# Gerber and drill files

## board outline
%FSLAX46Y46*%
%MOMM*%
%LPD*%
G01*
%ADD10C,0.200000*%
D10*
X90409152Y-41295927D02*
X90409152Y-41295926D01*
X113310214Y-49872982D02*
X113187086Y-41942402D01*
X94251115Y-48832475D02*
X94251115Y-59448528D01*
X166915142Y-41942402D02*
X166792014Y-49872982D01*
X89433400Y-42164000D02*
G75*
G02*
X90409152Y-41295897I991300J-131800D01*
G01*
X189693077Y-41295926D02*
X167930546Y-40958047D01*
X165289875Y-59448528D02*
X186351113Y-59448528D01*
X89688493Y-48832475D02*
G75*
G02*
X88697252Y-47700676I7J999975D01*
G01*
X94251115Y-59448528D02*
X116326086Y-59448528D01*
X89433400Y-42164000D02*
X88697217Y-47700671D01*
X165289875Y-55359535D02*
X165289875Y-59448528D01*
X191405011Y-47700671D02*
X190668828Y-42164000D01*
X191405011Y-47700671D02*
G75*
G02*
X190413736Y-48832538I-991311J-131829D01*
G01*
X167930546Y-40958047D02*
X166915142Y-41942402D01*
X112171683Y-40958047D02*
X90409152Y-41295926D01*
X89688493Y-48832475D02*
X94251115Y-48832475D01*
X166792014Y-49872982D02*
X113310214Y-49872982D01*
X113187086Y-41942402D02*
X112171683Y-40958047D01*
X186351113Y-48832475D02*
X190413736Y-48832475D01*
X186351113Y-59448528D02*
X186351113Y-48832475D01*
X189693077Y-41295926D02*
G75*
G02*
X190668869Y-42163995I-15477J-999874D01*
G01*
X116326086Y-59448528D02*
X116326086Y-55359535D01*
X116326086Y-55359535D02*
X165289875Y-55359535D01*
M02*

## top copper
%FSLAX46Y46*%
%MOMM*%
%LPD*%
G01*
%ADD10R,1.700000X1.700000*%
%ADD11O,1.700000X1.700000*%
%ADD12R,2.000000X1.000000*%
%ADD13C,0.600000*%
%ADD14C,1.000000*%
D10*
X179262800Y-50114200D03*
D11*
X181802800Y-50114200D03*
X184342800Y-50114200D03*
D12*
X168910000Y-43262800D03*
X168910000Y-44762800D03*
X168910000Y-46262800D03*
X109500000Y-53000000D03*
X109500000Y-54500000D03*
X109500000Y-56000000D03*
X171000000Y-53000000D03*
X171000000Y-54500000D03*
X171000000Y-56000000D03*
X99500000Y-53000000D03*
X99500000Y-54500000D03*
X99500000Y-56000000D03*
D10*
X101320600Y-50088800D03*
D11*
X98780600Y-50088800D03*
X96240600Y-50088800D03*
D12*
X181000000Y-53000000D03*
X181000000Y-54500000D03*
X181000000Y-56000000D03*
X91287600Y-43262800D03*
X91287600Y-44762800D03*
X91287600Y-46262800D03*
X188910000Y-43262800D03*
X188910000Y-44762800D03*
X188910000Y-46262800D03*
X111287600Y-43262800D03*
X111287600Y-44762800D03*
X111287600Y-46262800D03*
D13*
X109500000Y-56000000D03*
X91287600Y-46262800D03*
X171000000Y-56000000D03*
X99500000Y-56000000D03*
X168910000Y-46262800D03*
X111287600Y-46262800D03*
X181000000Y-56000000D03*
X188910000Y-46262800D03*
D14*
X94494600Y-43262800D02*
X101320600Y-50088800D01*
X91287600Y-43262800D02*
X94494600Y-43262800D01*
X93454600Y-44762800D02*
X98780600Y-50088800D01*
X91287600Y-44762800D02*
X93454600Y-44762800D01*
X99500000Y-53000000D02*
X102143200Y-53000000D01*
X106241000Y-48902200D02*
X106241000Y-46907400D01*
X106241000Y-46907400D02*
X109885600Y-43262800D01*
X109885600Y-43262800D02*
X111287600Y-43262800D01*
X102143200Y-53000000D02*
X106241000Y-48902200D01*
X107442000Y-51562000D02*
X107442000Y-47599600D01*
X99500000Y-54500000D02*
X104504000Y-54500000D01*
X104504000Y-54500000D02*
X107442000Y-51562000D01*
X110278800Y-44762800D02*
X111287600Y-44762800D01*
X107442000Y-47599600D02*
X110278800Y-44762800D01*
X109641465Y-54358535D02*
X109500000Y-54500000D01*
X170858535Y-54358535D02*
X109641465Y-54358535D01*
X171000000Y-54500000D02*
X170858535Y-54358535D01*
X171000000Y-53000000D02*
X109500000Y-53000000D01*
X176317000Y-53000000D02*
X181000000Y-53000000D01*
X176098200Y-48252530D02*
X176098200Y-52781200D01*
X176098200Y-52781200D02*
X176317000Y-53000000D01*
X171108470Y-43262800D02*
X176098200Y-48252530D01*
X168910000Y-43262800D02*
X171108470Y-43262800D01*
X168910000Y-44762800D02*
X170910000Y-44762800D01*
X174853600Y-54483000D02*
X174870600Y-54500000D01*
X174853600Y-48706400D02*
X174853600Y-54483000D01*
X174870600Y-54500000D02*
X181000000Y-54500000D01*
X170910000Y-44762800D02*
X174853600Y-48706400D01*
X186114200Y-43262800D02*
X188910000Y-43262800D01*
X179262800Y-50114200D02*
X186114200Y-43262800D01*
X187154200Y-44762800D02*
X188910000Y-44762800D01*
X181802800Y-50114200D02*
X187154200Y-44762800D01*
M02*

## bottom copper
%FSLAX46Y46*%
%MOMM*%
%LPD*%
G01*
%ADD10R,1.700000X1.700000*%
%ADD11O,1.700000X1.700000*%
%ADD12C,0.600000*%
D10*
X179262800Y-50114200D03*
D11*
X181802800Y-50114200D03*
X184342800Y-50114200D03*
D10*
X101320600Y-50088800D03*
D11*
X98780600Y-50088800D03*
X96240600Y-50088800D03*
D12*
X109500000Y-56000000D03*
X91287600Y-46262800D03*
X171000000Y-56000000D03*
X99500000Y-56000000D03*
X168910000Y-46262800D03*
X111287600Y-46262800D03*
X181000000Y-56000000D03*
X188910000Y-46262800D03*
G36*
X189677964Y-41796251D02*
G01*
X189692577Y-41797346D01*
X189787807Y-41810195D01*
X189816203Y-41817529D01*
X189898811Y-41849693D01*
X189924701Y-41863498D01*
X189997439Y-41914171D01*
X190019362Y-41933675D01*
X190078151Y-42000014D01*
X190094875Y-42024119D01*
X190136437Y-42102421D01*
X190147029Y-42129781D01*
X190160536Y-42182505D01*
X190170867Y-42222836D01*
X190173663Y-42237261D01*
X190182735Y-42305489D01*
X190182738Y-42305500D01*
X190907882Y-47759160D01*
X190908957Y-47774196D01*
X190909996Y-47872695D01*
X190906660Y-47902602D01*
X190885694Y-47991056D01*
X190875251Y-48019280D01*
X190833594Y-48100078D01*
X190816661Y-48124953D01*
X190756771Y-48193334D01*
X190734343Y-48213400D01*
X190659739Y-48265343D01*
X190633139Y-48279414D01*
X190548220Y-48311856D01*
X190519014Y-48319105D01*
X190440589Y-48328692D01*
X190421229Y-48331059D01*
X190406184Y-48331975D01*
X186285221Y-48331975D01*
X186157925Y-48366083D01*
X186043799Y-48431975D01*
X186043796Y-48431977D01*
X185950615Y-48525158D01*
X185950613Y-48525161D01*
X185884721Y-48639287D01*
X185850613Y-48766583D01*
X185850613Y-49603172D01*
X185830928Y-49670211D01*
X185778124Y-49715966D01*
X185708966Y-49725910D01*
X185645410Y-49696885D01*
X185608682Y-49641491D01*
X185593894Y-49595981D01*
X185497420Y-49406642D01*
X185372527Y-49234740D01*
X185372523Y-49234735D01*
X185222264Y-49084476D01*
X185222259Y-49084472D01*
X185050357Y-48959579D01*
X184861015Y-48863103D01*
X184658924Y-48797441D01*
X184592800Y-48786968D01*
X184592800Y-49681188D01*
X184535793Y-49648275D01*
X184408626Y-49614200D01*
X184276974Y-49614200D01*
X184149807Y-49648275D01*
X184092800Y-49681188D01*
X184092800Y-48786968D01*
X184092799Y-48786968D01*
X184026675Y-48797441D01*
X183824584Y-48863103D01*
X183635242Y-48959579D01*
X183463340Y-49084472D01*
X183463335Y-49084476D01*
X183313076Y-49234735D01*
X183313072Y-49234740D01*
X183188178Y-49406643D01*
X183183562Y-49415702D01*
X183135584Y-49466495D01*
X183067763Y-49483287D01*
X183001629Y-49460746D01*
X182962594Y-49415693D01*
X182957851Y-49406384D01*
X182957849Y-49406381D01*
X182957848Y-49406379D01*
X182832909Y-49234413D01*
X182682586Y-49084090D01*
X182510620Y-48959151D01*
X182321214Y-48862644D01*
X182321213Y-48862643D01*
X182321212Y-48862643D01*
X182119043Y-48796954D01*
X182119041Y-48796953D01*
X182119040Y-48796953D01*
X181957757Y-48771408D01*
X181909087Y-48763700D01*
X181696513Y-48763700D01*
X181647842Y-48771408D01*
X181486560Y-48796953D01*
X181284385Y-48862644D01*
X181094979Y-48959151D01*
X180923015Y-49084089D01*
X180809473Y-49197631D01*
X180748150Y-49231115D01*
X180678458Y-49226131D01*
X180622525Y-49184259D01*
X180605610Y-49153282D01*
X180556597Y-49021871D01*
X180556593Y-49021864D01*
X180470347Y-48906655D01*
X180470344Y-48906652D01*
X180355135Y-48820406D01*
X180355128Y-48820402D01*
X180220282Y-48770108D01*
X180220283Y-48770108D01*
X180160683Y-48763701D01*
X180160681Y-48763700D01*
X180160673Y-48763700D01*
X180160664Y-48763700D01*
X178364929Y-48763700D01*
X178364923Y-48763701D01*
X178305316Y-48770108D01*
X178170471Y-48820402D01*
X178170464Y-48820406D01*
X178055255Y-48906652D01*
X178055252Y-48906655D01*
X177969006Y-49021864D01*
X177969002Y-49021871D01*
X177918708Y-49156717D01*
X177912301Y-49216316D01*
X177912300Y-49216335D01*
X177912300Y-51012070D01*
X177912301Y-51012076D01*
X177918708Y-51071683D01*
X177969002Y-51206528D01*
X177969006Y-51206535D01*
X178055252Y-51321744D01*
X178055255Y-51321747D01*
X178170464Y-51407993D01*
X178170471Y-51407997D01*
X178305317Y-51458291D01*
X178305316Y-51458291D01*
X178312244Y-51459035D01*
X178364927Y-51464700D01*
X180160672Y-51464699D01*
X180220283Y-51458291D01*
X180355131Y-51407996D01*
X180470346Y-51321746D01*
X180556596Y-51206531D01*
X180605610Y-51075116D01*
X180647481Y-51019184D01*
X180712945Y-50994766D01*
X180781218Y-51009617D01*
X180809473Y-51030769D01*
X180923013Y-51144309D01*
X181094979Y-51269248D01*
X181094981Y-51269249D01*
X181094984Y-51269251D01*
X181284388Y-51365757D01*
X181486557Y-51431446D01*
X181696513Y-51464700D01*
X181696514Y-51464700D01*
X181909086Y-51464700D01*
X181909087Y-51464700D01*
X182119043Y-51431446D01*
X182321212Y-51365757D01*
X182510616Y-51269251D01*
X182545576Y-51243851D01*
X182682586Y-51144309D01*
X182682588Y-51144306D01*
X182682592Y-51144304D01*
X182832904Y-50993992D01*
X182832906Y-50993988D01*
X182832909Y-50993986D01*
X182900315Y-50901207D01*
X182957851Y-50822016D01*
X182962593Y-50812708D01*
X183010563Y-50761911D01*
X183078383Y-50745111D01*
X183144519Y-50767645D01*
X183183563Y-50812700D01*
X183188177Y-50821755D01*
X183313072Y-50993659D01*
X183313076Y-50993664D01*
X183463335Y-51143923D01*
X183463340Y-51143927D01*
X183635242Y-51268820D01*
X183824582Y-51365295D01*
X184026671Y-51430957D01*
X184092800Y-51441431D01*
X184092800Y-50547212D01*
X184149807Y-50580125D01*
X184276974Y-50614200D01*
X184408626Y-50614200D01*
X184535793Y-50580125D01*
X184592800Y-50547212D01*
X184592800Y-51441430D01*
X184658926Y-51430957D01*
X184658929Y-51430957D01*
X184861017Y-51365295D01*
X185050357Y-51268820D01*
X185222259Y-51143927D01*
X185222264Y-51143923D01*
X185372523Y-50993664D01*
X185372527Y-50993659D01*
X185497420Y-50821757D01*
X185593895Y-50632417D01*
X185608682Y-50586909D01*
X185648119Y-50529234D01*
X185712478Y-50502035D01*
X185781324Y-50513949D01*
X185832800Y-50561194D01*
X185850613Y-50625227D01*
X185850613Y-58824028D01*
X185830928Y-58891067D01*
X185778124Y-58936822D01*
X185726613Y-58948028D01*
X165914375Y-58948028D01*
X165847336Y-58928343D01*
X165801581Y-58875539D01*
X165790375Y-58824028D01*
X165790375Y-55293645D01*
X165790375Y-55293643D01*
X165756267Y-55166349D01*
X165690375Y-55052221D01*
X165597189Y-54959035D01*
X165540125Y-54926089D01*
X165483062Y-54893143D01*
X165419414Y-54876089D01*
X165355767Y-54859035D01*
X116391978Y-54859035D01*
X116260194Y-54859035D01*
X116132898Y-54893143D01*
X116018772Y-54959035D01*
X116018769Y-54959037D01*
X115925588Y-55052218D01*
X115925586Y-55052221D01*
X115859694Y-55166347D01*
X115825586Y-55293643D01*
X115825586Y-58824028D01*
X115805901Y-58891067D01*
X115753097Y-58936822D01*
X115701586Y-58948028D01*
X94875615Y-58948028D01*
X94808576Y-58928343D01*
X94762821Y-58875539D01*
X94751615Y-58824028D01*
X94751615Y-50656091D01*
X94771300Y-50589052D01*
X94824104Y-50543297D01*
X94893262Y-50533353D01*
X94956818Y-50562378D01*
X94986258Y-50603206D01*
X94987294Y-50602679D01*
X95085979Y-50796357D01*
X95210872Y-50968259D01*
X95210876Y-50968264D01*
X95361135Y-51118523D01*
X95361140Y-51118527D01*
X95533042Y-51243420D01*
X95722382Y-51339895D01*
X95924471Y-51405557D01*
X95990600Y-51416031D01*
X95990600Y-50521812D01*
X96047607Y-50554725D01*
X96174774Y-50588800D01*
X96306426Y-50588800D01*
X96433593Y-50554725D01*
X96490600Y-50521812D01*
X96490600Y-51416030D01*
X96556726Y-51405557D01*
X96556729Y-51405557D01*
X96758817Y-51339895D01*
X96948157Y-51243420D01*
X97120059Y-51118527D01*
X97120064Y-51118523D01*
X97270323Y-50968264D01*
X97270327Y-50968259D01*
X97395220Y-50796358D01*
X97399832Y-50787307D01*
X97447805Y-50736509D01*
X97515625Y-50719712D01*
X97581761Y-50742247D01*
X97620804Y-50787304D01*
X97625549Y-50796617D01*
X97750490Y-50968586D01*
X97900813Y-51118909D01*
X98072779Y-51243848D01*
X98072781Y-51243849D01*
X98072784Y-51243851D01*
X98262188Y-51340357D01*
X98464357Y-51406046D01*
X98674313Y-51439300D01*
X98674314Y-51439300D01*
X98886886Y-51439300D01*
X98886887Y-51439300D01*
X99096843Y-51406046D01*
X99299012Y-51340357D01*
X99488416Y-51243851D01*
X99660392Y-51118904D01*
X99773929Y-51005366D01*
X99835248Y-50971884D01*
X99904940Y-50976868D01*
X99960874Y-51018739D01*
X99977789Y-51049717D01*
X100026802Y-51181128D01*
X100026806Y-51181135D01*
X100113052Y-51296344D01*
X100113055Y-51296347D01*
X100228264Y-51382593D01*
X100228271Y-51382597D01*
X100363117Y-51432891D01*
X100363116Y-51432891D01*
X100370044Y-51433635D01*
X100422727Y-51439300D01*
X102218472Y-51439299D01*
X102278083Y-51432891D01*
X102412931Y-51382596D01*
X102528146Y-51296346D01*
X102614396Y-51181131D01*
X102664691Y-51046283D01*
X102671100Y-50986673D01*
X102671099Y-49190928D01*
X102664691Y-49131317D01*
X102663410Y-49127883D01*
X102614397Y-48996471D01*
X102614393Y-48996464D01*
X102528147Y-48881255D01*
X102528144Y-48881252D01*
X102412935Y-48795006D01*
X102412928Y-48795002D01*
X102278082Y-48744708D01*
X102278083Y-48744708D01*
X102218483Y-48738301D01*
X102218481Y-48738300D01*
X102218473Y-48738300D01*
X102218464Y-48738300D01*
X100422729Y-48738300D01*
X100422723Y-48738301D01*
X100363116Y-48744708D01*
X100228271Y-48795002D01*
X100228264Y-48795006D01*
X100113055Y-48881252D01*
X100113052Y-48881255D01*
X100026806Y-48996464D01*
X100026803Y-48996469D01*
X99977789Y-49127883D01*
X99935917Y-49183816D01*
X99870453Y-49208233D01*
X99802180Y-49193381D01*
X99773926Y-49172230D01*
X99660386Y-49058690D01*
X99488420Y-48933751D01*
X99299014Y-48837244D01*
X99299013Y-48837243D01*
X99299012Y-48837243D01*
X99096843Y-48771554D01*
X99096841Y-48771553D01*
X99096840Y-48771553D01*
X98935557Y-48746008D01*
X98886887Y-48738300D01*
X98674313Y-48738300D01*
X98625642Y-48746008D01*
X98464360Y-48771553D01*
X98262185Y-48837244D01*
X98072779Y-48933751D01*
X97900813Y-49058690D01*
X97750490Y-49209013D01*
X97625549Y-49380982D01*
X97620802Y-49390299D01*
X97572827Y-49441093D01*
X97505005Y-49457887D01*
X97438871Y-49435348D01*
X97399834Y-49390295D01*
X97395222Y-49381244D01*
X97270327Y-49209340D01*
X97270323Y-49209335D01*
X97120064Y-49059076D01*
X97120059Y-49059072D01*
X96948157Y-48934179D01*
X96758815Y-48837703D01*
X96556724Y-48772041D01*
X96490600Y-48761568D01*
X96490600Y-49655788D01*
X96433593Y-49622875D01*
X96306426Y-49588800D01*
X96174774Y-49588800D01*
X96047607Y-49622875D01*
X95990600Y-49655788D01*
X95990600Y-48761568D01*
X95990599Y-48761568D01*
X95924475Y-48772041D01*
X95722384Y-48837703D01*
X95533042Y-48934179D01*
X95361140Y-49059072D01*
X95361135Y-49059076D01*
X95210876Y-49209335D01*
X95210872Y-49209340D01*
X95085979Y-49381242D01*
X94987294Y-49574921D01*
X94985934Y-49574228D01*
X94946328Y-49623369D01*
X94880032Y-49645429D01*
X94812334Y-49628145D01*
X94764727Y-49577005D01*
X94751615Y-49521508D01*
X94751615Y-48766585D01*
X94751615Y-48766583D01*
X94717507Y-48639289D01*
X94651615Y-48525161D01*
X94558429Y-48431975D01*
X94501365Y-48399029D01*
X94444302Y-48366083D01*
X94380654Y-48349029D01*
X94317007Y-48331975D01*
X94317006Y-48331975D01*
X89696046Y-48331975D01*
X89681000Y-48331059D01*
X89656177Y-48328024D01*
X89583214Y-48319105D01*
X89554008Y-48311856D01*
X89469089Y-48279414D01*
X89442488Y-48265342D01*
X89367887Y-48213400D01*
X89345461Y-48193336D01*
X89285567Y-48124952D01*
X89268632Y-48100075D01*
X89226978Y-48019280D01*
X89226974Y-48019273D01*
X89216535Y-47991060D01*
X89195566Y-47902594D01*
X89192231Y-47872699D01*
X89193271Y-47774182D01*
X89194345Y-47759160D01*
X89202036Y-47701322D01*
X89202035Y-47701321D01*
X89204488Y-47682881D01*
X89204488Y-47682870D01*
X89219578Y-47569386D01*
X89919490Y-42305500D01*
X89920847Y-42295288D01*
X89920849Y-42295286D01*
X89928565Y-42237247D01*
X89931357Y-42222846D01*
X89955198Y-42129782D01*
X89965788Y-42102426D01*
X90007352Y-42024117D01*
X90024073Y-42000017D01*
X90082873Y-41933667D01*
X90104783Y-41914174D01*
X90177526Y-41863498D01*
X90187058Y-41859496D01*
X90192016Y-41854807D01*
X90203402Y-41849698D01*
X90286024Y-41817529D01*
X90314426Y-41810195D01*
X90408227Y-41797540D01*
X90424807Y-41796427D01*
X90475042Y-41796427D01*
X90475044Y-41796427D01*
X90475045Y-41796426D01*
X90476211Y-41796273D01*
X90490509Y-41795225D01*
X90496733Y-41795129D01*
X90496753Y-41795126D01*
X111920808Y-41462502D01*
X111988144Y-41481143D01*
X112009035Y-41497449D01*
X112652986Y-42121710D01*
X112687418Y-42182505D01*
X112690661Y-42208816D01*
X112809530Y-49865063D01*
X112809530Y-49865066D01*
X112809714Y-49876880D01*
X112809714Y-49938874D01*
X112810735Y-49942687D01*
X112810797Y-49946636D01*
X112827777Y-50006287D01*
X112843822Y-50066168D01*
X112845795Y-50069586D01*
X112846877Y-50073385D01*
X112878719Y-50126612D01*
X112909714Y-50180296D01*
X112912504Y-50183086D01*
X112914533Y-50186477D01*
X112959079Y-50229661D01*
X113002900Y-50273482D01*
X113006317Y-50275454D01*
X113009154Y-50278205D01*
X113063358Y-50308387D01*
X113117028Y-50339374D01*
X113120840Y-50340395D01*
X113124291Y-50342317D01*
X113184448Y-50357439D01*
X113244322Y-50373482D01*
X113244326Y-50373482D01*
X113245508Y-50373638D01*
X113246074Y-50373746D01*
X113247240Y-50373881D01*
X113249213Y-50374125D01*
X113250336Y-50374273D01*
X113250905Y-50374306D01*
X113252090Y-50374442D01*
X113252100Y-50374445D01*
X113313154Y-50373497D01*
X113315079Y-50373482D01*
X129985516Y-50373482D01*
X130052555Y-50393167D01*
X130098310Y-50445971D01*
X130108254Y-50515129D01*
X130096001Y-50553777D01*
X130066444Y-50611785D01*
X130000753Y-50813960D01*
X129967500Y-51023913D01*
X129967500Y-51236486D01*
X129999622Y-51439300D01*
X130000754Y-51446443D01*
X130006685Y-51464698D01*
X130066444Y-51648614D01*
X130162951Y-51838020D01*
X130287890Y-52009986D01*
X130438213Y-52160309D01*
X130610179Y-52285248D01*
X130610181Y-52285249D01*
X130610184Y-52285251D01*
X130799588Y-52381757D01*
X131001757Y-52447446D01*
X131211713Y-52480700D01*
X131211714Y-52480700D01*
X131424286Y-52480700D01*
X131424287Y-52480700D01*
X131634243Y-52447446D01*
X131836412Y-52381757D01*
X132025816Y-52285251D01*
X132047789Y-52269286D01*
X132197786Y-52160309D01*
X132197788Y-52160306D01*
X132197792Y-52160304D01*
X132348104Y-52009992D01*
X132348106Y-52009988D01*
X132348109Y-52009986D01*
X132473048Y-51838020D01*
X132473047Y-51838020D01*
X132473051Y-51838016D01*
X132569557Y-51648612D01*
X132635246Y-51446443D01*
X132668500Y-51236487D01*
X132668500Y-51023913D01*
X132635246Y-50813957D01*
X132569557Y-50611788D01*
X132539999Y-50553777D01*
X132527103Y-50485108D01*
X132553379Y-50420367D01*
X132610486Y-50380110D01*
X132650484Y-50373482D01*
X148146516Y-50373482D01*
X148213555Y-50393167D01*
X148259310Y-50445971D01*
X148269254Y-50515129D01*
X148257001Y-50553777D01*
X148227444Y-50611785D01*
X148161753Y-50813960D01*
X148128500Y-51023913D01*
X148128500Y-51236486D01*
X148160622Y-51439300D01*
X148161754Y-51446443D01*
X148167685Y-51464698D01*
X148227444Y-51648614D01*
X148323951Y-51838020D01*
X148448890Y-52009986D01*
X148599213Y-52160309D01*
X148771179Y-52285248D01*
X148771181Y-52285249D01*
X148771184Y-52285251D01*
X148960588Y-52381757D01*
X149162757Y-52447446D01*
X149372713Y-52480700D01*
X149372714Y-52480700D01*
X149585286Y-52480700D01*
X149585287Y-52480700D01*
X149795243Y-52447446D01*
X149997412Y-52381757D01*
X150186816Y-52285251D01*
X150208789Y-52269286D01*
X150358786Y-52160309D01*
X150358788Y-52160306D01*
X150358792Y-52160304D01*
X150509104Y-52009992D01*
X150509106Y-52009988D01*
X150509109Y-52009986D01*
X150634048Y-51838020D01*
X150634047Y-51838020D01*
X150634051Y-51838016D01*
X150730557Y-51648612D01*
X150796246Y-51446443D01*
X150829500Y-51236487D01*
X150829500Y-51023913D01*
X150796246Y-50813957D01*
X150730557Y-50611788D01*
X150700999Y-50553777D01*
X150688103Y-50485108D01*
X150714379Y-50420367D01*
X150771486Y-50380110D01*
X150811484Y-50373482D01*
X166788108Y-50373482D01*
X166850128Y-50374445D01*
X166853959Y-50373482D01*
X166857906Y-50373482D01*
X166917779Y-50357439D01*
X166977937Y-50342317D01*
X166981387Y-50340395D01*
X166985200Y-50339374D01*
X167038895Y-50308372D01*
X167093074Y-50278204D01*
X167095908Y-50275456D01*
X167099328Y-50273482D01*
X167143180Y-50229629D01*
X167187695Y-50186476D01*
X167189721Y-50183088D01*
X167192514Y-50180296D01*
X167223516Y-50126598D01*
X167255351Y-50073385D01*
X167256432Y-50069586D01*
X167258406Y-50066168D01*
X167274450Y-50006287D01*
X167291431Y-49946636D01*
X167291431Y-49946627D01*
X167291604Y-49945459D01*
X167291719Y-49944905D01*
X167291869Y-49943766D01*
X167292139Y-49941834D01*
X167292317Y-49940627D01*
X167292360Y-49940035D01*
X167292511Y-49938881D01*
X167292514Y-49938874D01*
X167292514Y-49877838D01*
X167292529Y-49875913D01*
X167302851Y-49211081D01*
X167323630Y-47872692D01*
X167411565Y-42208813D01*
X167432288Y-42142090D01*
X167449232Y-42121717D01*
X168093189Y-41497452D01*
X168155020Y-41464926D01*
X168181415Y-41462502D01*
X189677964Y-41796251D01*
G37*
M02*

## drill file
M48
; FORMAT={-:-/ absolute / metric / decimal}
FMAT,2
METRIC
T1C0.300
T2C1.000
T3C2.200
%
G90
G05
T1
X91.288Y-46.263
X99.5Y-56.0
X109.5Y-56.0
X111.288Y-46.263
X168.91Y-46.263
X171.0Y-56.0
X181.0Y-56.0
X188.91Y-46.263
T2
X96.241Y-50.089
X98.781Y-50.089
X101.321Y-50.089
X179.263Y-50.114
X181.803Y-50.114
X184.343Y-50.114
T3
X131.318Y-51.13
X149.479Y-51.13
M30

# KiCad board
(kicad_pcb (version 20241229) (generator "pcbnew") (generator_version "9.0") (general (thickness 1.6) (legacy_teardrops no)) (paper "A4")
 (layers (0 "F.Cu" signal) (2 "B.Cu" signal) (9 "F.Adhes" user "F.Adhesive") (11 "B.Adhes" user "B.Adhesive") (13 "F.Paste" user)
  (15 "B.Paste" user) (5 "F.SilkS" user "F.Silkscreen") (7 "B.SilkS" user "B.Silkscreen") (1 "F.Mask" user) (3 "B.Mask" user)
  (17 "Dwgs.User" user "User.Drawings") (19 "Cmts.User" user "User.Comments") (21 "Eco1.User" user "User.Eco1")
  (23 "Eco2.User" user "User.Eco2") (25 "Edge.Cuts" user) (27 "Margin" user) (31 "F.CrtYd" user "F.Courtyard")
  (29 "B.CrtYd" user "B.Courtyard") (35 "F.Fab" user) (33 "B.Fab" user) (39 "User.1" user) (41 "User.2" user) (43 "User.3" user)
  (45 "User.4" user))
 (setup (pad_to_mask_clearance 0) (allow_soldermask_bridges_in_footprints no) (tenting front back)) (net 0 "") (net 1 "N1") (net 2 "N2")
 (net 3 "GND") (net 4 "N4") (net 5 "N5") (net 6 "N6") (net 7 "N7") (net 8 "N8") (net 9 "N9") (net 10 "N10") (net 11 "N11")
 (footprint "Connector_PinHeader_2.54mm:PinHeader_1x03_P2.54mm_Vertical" (layer "F.Cu") (at 179.2628 50.1142 90)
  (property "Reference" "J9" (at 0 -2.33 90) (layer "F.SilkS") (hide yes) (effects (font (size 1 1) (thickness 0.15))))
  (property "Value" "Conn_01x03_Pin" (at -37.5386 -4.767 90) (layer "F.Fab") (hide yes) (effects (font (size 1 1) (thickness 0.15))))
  (pad "1" thru_hole rect (at 0 0 90) (size 1.7 1.7) (drill 1) (layers "*.Cu" "*.Mask") (remove_unused_layers no) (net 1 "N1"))
  (pad "2" thru_hole oval (at 0 2.54 90) (size 1.7 1.7) (drill 1) (layers "*.Cu" "*.Mask") (remove_unused_layers no) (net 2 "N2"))
  (pad "3" thru_hole oval (at 0 5.08 90) (size 1.7 1.7) (drill 1) (layers "*.Cu" "*.Mask") (remove_unused_layers no) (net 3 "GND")))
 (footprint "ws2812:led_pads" (layer "F.Cu") (at 168.91 44.7628 -90)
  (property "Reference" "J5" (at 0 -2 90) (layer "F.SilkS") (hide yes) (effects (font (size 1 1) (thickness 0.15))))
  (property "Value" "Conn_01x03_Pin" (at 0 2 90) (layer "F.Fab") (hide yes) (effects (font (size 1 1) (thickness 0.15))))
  (pad "1" smd rect (at -1.5 0 270) (size 1 2) (layers "F.Cu" "F.Mask" "F.Paste") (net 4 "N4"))
  (pad "2" smd rect (at 0 0 270) (size 1 2) (layers "F.Cu" "F.Mask" "F.Paste") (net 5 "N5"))
  (pad "3" smd rect (at 1.5 0 270) (size 1 2) (layers "F.Cu" "F.Mask" "F.Paste") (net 3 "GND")))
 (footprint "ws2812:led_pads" (layer "F.Cu") (at 109.5 54.5 -90)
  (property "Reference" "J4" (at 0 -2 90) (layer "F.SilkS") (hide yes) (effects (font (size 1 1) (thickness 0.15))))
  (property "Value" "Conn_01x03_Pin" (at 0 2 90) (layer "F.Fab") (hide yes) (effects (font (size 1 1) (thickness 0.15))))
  (pad "1" smd rect (at -1.5 0 270) (size 1 2) (layers "F.Cu" "F.Mask" "F.Paste") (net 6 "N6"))
  (pad "2" smd rect (at 0 0 270) (size 1 2) (layers "F.Cu" "F.Mask" "F.Paste") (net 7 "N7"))
  (pad "3" smd rect (at 1.5 0 270) (size 1 2) (layers "F.Cu" "F.Mask" "F.Paste") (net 3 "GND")))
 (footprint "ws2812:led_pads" (layer "F.Cu") (at 171 54.5 -90)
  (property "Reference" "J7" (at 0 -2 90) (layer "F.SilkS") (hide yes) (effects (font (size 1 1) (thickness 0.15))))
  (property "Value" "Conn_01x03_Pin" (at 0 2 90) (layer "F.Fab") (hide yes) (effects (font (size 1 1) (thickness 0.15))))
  (pad "1" smd rect (at -1.5 0 270) (size 1 2) (layers "F.Cu" "F.Mask" "F.Paste") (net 6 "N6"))
  (pad "2" smd rect (at 0 0 270) (size 1 2) (layers "F.Cu" "F.Mask" "F.Paste") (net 7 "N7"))
  (pad "3" smd rect (at 1.5 0 270) (size 1 2) (layers "F.Cu" "F.Mask" "F.Paste") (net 3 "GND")))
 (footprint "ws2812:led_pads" (layer "F.Cu") (at 99.5 54.5 -90)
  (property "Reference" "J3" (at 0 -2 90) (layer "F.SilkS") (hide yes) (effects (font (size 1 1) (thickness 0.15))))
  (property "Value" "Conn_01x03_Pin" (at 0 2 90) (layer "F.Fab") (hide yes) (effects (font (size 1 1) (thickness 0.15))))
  (pad "1" smd rect (at -1.5 0 270) (size 1 2) (layers "F.Cu" "F.Mask" "F.Paste") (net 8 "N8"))
  (pad "2" smd rect (at 0 0 270) (size 1 2) (layers "F.Cu" "F.Mask" "F.Paste") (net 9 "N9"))
  (pad "3" smd rect (at 1.5 0 270) (size 1 2) (layers "F.Cu" "F.Mask" "F.Paste") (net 3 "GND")))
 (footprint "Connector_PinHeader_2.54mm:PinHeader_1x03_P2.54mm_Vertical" (layer "F.Cu") (at 101.3206 50.0888 -90)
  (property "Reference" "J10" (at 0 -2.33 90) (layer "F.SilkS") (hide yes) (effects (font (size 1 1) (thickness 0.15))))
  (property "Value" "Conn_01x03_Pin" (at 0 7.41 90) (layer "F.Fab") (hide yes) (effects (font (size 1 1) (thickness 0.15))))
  (pad "1" thru_hole rect (at 0 0 270) (size 1.7 1.7) (drill 1) (layers "*.Cu" "*.Mask") (remove_unused_layers no) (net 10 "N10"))
  (pad "2" thru_hole oval (at 0 2.54 270) (size 1.7 1.7) (drill 1) (layers "*.Cu" "*.Mask") (remove_unused_layers no) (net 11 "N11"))
  (pad "3" thru_hole oval (at 0 5.08 270) (size 1.7 1.7) (drill 1) (layers "*.Cu" "*.Mask") (remove_unused_layers no) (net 3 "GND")))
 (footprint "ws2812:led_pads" (layer "F.Cu") (at 181 54.5 -90)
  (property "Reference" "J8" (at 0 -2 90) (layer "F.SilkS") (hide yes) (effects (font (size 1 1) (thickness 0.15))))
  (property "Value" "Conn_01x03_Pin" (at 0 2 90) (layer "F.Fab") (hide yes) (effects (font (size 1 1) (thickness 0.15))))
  (pad "1" smd rect (at -1.5 0 270) (size 1 2) (layers "F.Cu" "F.Mask" "F.Paste") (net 4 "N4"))
  (pad "2" smd rect (at 0 0 270) (size 1 2) (layers "F.Cu" "F.Mask" "F.Paste") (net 5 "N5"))
  (pad "3" smd rect (at 1.5 0 270) (size 1 2) (layers "F.Cu" "F.Mask" "F.Paste") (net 3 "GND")))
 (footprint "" (layer "F.Cu") (at 149.479 51.1302)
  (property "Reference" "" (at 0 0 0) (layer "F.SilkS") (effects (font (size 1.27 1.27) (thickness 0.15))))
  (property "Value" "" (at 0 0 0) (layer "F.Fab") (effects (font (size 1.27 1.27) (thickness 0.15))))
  (pad "" np_thru_hole circle (at 0 0) (size 2.2 2.2) (drill 2.2) (layers "*.Cu" "*.Mask")))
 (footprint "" (layer "F.Cu") (at 131.318 51.1302)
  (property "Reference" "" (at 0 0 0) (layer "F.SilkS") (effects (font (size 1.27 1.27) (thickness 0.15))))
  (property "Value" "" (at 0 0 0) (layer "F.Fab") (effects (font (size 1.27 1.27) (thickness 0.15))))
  (pad "" np_thru_hole circle (at 0 0) (size 2.2 2.2) (drill 2.2) (layers "*.Cu" "*.Mask")))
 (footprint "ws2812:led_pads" (layer "F.Cu") (at 91.2876 44.7628 -90)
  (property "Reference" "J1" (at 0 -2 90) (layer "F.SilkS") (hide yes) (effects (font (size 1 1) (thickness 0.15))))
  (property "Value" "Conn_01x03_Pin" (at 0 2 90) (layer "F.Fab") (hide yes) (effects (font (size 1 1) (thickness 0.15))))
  (pad "1" smd rect (at -1.5 0 270) (size 1 2) (layers "F.Cu" "F.Mask" "F.Paste") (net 10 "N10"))
  (pad "2" smd rect (at 0 0 270) (size 1 2) (layers "F.Cu" "F.Mask" "F.Paste") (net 11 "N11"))
  (pad "3" smd rect (at 1.5 0 270) (size 1 2) (layers "F.Cu" "F.Mask" "F.Paste") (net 3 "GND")))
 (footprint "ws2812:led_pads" (layer "F.Cu") (at 188.91 44.7628 -90)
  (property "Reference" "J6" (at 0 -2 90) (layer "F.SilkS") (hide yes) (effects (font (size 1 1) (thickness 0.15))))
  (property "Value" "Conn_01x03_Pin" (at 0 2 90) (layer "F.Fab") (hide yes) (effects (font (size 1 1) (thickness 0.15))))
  (pad "1" smd rect (at -1.5 0 270) (size 1 2) (layers "F.Cu" "F.Mask" "F.Paste") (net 1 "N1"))
  (pad "2" smd rect (at 0 0 270) (size 1 2) (layers "F.Cu" "F.Mask" "F.Paste") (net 2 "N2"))
  (pad "3" smd rect (at 1.5 0 270) (size 1 2) (layers "F.Cu" "F.Mask" "F.Paste") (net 3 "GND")))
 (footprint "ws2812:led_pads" (layer "F.Cu") (at 111.2876 44.7628 -90)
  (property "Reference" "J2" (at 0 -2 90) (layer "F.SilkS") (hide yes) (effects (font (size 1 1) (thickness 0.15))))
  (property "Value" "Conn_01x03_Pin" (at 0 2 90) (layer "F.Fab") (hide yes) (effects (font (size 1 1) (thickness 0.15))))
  (pad "1" smd rect (at -1.5 0 270) (size 1 2) (layers "F.Cu" "F.Mask" "F.Paste") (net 8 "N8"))
  (pad "2" smd rect (at 0 0 270) (size 1 2) (layers "F.Cu" "F.Mask" "F.Paste") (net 9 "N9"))
  (pad "3" smd rect (at 1.5 0 270) (size 1 2) (layers "F.Cu" "F.Mask" "F.Paste") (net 3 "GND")))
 (gr_line (start 90.409152 41.295927) (end 90.409152 41.295926) (stroke (width 0.2) (type default)) (layer "Edge.Cuts"))
 (gr_line (start 113.310214 49.872982) (end 113.187086 41.942402) (stroke (width 0.2) (type default)) (layer "Edge.Cuts"))
 (gr_line (start 94.251115 48.832475) (end 94.251115 59.448528) (stroke (width 0.2) (type default)) (layer "Edge.Cuts"))
 (gr_line (start 166.915142 41.942402) (end 166.792014 49.872982) (stroke (width 0.2) (type default)) (layer "Edge.Cuts"))
 (gr_arc (start 89.4334 42.164) (mid 89.759996 41.548677) (end 90.409152 41.295927) (stroke (width 0.2) (type default)) (layer "Edge.Cuts"))
 (gr_line (start 189.693077 41.295926) (end 167.930546 40.958047) (stroke (width 0.2) (type default)) (layer "Edge.Cuts"))
 (gr_line (start 165.289875 59.448528) (end 186.351113 59.448528) (stroke (width 0.2) (type default)) (layer "Edge.Cuts"))
 (gr_arc (start 89.688493 48.832475) (mid 88.936228 48.491336) (end 88.697217 47.700671) (stroke (width 0.2) (type default))
  (layer "Edge.Cuts"))
 (gr_line (start 94.251115 59.448528) (end 116.326086 59.448528) (stroke (width 0.2) (type default)) (layer "Edge.Cuts"))
 (gr_line (start 89.4334 42.164) (end 88.697217 47.700671) (stroke (width 0.2) (type default)) (layer "Edge.Cuts"))
 (gr_line (start 165.289875 55.359535) (end 165.289875 59.448528) (stroke (width 0.2) (type default)) (layer "Edge.Cuts"))
 (gr_line (start 191.405011 47.700671) (end 190.668828 42.164) (stroke (width 0.2) (type default)) (layer "Edge.Cuts"))
 (gr_arc (start 191.405011 47.700671) (mid 191.166001 48.491336) (end 190.413736 48.832475) (stroke (width 0.2) (type default))
  (layer "Edge.Cuts"))
 (gr_line (start 167.930546 40.958047) (end 166.915142 41.942402) (stroke (width 0.2) (type default)) (layer "Edge.Cuts"))
 (gr_line (start 112.171683 40.958047) (end 90.409152 41.295926) (stroke (width 0.2) (type default)) (layer "Edge.Cuts"))
 (gr_line (start 89.688493 48.832475) (end 94.251115 48.832475) (stroke (width 0.2) (type default)) (layer "Edge.Cuts"))
 (gr_line (start 166.792014 49.872982) (end 113.310214 49.872982) (stroke (width 0.2) (type default)) (layer "Edge.Cuts"))
 (gr_line (start 113.187086 41.942402) (end 112.171683 40.958047) (stroke (width 0.2) (type default)) (layer "Edge.Cuts"))
 (gr_line (start 186.351113 48.832475) (end 190.413736 48.832475) (stroke (width 0.2) (type default)) (layer "Edge.Cuts"))
 (gr_line (start 186.351113 59.448528) (end 186.351113 48.832475) (stroke (width 0.2) (type default)) (layer "Edge.Cuts"))
 (gr_arc (start 189.693077 41.295926) (mid 190.342233 41.548677) (end 190.668828 42.164) (stroke (width 0.2) (type default))
  (layer "Edge.Cuts"))
 (gr_line (start 116.326086 59.448528) (end 116.326086 55.359535) (stroke (width 0.2) (type default)) (layer "Edge.Cuts"))
 (gr_line (start 116.326086 55.359535) (end 165.289875 55.359535) (stroke (width 0.2) (type default)) (layer "Edge.Cuts"))
 (segment (start 94.4946 43.2628) (end 101.3206 50.0888) (width 1) (layer "F.Cu") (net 10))
 (segment (start 91.2876 43.2628) (end 94.4946 43.2628) (width 1) (layer "F.Cu") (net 10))
 (via (at 109.5 56) (size 0.6) (drill 0.3) (layers "F.Cu" "B.Cu") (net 3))
 (via (at 91.2876 46.2628) (size 0.6) (drill 0.3) (layers "F.Cu" "B.Cu") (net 3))
 (via (at 171 56) (size 0.6) (drill 0.3) (layers "F.Cu" "B.Cu") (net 3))
 (via (at 99.5 56) (size 0.6) (drill 0.3) (layers "F.Cu" "B.Cu") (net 3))
 (via (at 168.91 46.2628) (size 0.6) (drill 0.3) (layers "F.Cu" "B.Cu") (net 3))
 (via (at 111.2876 46.2628) (size 0.6) (drill 0.3) (layers "F.Cu" "B.Cu") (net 3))
 (via (at 181 56) (size 0.6) (drill 0.3) (layers "F.Cu" "B.Cu") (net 3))
 (via (at 188.91 46.2628) (size 0.6) (drill 0.3) (layers "F.Cu" "B.Cu") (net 3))
 (segment (start 93.4546 44.7628) (end 98.7806 50.0888) (width 1) (layer "F.Cu") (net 11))
 (segment (start 91.2876 44.7628) (end 93.4546 44.7628) (width 1) (layer "F.Cu") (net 11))
 (segment (start 99.5 53) (end 102.1432 53) (width 1) (layer "F.Cu") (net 8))
 (segment (start 106.241 48.9022) (end 106.241 46.9074) (width 1) (layer "F.Cu") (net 8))
 (segment (start 106.241 46.9074) (end 109.8856 43.2628) (width 1) (layer "F.Cu") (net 8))
 (segment (start 109.8856 43.2628) (end 111.2876 43.2628) (width 1) (layer "F.Cu") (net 8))
 (segment (start 102.1432 53) (end 106.241 48.9022) (width 1) (layer "F.Cu") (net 8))
 (segment (start 107.442 51.562) (end 107.442 47.5996) (width 1) (layer "F.Cu") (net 9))
 (segment (start 99.5 54.5) (end 104.504 54.5) (width 1) (layer "F.Cu") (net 9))
 (segment (start 104.504 54.5) (end 107.442 51.562) (width 1) (layer "F.Cu") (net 9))
 (segment (start 110.2788 44.7628) (end 111.2876 44.7628) (width 1) (layer "F.Cu") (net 9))
 (segment (start 107.442 47.5996) (end 110.2788 44.7628) (width 1) (layer "F.Cu") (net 9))
 (segment (start 109.641465 54.358535) (end 109.5 54.5) (width 1) (layer "F.Cu") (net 7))
 (segment (start 170.858535 54.358535) (end 109.641465 54.358535) (width 1) (layer "F.Cu") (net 7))
 (segment (start 171 54.5) (end 170.858535 54.358535) (width 1) (layer "F.Cu") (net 7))
 (segment (start 171 53) (end 109.5 53) (width 1) (layer "F.Cu") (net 6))
 (segment (start 176.317 53) (end 181 53) (width 1) (layer "F.Cu") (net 4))
 (segment (start 176.0982 48.25253) (end 176.0982 52.7812) (width 1) (layer "F.Cu") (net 4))
 (segment (start 176.0982 52.7812) (end 176.317 53) (width 1) (layer "F.Cu") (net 4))
 (segment (start 171.10847 43.2628) (end 176.0982 48.25253) (width 1) (layer "F.Cu") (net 4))
 (segment (start 168.91 43.2628) (end 171.10847 43.2628) (width 1) (layer "F.Cu") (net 4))
 (segment (start 168.91 44.7628) (end 170.91 44.7628) (width 1) (layer "F.Cu") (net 5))
 (segment (start 174.8536 54.483) (end 174.8706 54.5) (width 1) (layer "F.Cu") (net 5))
 (segment (start 174.8536 48.7064) (end 174.8536 54.483) (width 1) (layer "F.Cu") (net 5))
 (segment (start 174.8706 54.5) (end 181 54.5) (width 1) (layer "F.Cu") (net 5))
 (segment (start 170.91 44.7628) (end 174.8536 48.7064) (width 1) (layer "F.Cu") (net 5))
 (segment (start 186.1142 43.2628) (end 188.91 43.2628) (width 1) (layer "F.Cu") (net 1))
 (segment (start 179.2628 50.1142) (end 186.1142 43.2628) (width 1) (layer "F.Cu") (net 1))
 (segment (start 187.1542 44.7628) (end 188.91 44.7628) (width 1) (layer "F.Cu") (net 2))
 (segment (start 181.8028 50.1142) (end 187.1542 44.7628) (width 1) (layer "F.Cu") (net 2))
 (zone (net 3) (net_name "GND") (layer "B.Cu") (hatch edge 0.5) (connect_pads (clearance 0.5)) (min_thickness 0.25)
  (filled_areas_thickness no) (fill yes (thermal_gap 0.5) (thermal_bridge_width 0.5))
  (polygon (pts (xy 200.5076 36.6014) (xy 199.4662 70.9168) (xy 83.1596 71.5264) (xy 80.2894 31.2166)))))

